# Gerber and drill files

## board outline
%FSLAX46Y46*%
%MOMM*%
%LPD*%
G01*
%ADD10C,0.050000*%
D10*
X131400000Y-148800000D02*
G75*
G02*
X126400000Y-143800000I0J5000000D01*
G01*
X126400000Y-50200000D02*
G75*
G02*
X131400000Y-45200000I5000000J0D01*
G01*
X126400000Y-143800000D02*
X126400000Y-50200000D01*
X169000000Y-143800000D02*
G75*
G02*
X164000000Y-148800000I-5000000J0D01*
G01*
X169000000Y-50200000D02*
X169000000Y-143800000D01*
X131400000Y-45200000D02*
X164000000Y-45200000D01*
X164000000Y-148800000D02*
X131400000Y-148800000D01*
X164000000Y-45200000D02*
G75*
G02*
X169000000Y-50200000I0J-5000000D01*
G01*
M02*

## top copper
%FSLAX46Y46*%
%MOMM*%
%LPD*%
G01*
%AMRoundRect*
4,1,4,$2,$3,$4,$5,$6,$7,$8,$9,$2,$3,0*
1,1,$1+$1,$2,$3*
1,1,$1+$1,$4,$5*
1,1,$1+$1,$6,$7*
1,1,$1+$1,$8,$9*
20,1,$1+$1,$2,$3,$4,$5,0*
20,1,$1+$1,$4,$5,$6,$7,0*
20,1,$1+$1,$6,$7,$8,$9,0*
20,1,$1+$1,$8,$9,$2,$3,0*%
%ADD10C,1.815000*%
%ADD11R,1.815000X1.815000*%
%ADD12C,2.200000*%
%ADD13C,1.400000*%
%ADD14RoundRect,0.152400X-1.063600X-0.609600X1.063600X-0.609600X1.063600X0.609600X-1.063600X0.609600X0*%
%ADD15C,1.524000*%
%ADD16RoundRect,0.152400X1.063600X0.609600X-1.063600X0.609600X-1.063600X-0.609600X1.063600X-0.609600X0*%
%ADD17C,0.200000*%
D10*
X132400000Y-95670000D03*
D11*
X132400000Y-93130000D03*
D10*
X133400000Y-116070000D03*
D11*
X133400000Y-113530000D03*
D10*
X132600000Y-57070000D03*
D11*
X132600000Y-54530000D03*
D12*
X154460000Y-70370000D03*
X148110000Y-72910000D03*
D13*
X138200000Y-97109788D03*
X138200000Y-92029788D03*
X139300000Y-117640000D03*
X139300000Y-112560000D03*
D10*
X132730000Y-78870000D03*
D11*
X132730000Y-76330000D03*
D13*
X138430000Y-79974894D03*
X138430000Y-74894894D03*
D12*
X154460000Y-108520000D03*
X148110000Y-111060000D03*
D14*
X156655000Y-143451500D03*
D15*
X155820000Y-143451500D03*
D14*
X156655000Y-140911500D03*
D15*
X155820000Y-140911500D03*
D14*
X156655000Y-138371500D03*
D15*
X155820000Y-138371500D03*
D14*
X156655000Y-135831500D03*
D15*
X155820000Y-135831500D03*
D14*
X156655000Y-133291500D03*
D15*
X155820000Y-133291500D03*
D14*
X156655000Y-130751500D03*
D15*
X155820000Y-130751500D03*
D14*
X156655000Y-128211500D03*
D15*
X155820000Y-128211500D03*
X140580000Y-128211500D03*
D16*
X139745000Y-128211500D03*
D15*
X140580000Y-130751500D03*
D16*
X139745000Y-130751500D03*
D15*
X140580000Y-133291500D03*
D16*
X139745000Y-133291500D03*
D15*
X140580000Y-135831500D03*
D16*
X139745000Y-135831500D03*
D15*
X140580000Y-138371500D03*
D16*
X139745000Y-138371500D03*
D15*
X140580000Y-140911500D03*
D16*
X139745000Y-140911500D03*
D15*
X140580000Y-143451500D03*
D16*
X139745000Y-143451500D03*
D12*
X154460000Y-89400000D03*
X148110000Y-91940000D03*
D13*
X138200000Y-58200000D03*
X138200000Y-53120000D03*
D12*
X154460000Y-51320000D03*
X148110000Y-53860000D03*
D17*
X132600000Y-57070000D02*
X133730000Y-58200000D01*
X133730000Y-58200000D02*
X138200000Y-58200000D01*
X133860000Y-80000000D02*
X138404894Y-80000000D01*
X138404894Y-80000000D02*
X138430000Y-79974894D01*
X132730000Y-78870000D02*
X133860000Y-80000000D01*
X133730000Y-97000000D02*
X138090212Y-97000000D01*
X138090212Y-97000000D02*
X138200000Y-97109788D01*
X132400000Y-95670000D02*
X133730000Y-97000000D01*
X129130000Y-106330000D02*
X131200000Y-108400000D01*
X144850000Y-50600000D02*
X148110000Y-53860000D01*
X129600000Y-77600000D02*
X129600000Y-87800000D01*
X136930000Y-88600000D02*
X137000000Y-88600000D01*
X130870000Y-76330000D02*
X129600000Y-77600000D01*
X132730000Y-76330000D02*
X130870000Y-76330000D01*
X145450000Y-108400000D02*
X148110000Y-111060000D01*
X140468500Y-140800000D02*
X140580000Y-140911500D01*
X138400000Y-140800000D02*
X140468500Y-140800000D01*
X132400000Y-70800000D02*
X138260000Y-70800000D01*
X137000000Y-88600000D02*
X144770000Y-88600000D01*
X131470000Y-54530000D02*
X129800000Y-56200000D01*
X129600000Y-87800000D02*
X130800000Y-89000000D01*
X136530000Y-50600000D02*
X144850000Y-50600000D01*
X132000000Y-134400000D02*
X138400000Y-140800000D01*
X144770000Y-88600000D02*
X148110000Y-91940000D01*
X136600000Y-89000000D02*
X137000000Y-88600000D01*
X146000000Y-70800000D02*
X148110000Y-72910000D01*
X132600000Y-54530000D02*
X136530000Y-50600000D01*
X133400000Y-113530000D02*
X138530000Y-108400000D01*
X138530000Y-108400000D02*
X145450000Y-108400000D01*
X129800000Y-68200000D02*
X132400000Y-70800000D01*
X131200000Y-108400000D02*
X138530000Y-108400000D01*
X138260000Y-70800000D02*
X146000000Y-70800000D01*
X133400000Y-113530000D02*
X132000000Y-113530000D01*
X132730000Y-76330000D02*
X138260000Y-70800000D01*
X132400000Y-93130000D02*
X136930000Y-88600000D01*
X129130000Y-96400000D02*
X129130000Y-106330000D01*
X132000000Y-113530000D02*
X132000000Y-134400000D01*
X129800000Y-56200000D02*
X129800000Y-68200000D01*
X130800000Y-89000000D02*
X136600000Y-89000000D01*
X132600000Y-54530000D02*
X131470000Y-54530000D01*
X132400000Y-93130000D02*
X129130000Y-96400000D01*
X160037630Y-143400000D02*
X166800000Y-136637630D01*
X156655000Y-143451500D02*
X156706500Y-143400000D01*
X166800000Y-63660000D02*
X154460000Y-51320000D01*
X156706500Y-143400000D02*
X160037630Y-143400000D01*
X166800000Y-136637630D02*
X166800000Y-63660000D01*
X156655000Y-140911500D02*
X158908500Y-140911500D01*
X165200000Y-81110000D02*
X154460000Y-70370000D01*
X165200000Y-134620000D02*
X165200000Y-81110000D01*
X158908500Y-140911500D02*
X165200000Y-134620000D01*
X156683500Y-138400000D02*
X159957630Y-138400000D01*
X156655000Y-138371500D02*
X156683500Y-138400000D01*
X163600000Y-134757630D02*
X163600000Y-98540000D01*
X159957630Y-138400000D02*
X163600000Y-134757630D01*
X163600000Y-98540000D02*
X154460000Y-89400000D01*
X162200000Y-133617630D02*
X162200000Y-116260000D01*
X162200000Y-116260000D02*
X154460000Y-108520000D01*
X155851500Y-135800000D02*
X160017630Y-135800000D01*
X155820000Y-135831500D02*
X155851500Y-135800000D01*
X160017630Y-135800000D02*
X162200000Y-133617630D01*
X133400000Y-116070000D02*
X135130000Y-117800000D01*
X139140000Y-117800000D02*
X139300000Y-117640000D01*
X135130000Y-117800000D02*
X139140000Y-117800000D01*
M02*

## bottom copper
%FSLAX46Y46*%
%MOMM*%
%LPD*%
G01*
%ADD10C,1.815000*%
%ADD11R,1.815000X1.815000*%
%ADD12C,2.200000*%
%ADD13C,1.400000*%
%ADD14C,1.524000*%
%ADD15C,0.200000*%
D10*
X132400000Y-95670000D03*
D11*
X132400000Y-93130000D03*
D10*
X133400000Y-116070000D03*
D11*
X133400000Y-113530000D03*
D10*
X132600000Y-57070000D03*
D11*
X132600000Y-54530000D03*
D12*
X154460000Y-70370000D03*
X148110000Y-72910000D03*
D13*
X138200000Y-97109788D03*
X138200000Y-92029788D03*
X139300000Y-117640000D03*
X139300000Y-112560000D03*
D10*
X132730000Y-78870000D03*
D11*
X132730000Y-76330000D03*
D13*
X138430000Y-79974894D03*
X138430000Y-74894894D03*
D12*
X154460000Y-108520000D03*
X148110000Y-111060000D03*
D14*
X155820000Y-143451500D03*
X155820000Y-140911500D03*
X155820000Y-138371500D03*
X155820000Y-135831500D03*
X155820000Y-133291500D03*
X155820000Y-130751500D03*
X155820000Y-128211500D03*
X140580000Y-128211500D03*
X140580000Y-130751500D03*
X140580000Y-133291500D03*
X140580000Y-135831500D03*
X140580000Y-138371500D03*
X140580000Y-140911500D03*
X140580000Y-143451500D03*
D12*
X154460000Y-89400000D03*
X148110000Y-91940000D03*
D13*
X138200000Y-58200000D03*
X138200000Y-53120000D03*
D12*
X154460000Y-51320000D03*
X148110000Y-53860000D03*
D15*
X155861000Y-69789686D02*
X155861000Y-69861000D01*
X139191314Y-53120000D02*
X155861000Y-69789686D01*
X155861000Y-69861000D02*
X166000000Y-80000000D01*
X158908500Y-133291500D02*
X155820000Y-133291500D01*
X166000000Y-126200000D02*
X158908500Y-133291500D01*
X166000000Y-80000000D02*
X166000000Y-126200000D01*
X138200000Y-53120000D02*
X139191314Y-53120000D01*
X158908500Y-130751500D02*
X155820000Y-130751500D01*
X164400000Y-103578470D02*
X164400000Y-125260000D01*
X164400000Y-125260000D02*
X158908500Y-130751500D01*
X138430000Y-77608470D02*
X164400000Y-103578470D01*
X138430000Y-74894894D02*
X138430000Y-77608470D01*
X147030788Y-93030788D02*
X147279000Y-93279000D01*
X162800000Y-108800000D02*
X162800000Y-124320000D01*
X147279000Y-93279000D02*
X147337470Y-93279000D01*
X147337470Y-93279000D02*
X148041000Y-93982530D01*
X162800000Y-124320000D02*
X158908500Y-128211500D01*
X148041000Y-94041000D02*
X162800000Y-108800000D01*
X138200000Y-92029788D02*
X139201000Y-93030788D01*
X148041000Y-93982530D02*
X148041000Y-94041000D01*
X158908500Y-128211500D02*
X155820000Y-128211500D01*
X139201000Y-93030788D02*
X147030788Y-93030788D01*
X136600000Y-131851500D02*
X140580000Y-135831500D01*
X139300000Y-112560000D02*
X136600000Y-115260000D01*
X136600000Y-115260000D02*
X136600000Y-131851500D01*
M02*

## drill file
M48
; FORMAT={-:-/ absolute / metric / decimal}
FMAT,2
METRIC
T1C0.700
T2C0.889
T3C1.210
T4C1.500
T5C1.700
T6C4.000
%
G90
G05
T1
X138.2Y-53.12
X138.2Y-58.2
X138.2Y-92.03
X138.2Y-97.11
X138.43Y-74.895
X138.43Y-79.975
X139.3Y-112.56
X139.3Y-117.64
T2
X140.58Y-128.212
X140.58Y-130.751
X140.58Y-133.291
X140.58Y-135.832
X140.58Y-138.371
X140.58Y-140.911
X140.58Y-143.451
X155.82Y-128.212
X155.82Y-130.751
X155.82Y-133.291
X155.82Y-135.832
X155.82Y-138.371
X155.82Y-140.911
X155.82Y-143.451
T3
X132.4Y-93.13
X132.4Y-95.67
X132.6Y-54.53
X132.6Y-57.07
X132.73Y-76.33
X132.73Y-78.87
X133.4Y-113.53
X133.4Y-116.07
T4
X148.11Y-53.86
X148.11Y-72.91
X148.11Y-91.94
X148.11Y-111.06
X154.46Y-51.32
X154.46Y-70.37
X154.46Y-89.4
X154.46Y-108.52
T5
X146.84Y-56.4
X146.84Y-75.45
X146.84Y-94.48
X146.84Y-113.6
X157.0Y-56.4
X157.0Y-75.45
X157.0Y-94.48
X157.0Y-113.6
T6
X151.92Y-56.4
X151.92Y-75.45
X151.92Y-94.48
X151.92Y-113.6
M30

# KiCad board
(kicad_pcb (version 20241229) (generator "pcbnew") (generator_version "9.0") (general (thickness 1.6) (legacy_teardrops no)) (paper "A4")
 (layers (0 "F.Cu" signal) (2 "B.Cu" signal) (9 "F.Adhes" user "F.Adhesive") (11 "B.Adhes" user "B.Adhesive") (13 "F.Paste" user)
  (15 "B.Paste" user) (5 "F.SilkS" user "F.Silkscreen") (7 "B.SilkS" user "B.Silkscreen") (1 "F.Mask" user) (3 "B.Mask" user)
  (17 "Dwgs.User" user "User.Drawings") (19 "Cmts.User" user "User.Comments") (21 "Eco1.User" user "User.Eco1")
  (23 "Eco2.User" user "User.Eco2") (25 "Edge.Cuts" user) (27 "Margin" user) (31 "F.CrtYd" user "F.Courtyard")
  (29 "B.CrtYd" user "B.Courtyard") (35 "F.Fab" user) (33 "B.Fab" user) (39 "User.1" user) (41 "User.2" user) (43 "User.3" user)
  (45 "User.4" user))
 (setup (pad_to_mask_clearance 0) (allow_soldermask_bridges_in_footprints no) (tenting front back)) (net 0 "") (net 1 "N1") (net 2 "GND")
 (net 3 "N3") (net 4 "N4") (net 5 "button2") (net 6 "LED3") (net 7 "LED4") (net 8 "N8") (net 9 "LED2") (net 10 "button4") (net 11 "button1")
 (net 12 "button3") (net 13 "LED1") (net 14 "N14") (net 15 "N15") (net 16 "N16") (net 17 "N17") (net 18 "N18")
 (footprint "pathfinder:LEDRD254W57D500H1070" (layer "F.Cu") (at 132.4 94.4 -90)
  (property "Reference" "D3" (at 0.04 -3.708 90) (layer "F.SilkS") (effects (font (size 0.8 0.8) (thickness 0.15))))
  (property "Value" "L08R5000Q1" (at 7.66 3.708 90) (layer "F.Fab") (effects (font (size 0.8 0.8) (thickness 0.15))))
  (pad "A" thru_hole circle (at 1.27 0 270) (size 1.815 1.815) (drill 1.21) (layers "*.Cu" "*.Mask") (remove_unused_layers no) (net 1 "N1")
   (solder_mask_margin 0.102))
  (pad "C" thru_hole rect (at -1.27 0 270) (size 1.815 1.815) (drill 1.21) (layers "*.Cu" "*.Mask") (remove_unused_layers no) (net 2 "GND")
   (solder_mask_margin 0.102)))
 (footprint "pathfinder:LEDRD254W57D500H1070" (layer "F.Cu") (at 133.4 114.8 -90)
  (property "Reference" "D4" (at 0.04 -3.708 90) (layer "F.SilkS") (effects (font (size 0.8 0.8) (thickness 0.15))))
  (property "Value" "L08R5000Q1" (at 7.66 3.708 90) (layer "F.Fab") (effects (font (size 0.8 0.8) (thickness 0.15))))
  (pad "A" thru_hole circle (at 1.27 0 270) (size 1.815 1.815) (drill 1.21) (layers "*.Cu" "*.Mask") (remove_unused_layers no) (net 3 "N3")
   (solder_mask_margin 0.102))
  (pad "C" thru_hole rect (at -1.27 0 270) (size 1.815 1.815) (drill 1.21) (layers "*.Cu" "*.Mask") (remove_unused_layers no) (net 2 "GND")
   (solder_mask_margin 0.102)))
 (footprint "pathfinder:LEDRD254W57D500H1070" (layer "F.Cu") (at 132.6 55.8 -90)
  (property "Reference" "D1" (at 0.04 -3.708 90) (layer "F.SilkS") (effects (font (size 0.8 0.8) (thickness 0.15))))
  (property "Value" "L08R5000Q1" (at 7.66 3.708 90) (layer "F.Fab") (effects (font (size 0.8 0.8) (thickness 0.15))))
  (pad "A" thru_hole circle (at 1.27 0 270) (size 1.815 1.815) (drill 1.21) (layers "*.Cu" "*.Mask") (remove_unused_layers no) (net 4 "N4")
   (solder_mask_margin 0.102))
  (pad "C" thru_hole rect (at -1.27 0 270) (size 1.815 1.815) (drill 1.21) (layers "*.Cu" "*.Mask") (remove_unused_layers no) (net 2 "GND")
   (solder_mask_margin 0.102)))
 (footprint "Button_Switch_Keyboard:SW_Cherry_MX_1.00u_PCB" (layer "F.Cu") (at 154.46 70.37)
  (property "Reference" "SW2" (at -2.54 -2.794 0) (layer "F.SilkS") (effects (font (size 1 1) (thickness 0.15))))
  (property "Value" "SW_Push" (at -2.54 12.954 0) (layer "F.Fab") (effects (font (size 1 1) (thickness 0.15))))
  (pad "" np_thru_hole circle (at -7.62 5.08) (size 1.7 1.7) (drill 1.7) (layers "*.Cu" "*.Mask"))
  (pad "" np_thru_hole circle (at -2.54 5.08) (size 4 4) (drill 4) (layers "*.Cu" "*.Mask"))
  (pad "" np_thru_hole circle (at 2.54 5.08) (size 1.7 1.7) (drill 1.7) (layers "*.Cu" "*.Mask"))
  (pad "1" thru_hole circle (at 0 0) (size 2.2 2.2) (drill 1.5) (layers "*.Cu" "*.Mask") (remove_unused_layers no) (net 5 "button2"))
  (pad "2" thru_hole circle (at -6.35 2.54) (size 2.2 2.2) (drill 1.5) (layers "*.Cu" "*.Mask") (remove_unused_layers no) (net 2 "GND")))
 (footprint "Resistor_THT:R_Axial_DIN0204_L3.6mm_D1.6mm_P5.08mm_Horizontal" (layer "F.Cu") (at 138.2 97.109788 90)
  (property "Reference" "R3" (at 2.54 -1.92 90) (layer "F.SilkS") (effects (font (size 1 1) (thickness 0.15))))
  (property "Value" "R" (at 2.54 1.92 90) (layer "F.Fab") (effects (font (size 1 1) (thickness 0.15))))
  (pad "1" thru_hole circle (at 0 0 90) (size 1.4 1.4) (drill 0.7) (layers "*.Cu" "*.Mask") (remove_unused_layers no) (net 1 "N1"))
  (pad "2" thru_hole circle (at 5.08 0 90) (size 1.4 1.4) (drill 0.7) (layers "*.Cu" "*.Mask") (remove_unused_layers no) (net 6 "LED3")))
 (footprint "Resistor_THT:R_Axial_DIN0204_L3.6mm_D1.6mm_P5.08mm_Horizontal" (layer "F.Cu") (at 139.3 117.64 90)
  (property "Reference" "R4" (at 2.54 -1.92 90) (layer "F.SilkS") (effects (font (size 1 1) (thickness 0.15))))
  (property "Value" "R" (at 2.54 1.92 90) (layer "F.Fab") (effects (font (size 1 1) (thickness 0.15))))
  (pad "1" thru_hole circle (at 0 0 90) (size 1.4 1.4) (drill 0.7) (layers "*.Cu" "*.Mask") (remove_unused_layers no) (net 3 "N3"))
  (pad "2" thru_hole circle (at 5.08 0 90) (size 1.4 1.4) (drill 0.7) (layers "*.Cu" "*.Mask") (remove_unused_layers no) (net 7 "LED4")))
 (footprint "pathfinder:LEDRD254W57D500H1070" (layer "F.Cu") (at 132.73 77.6 -90)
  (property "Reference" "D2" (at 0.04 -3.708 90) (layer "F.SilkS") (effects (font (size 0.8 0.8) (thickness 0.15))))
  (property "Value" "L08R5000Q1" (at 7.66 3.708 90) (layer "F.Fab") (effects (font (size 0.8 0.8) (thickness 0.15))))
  (pad "A" thru_hole circle (at 1.27 0 270) (size 1.815 1.815) (drill 1.21) (layers "*.Cu" "*.Mask") (remove_unused_layers no) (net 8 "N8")
   (solder_mask_margin 0.102))
  (pad "C" thru_hole rect (at -1.27 0 270) (size 1.815 1.815) (drill 1.21) (layers "*.Cu" "*.Mask") (remove_unused_layers no) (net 2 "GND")
   (solder_mask_margin 0.102)))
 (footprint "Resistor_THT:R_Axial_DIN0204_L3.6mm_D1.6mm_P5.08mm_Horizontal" (layer "F.Cu") (at 138.43 79.974894 90)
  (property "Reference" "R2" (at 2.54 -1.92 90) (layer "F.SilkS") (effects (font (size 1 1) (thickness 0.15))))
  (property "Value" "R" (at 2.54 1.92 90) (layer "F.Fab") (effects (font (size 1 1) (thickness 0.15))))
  (pad "1" thru_hole circle (at 0 0 90) (size 1.4 1.4) (drill 0.7) (layers "*.Cu" "*.Mask") (remove_unused_layers no) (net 8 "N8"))
  (pad "2" thru_hole circle (at 5.08 0 90) (size 1.4 1.4) (drill 0.7) (layers "*.Cu" "*.Mask") (remove_unused_layers no) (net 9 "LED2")))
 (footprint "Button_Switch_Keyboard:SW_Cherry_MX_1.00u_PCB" (layer "F.Cu") (at 154.46 108.52)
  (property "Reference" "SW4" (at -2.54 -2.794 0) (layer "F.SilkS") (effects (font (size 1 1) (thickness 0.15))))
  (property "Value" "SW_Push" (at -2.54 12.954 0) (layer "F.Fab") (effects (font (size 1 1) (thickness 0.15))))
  (pad "" np_thru_hole circle (at -7.62 5.08) (size 1.7 1.7) (drill 1.7) (layers "*.Cu" "*.Mask"))
  (pad "" np_thru_hole circle (at -2.54 5.08) (size 4 4) (drill 4) (layers "*.Cu" "*.Mask"))
  (pad "" np_thru_hole circle (at 2.54 5.08) (size 1.7 1.7) (drill 1.7) (layers "*.Cu" "*.Mask"))
  (pad "1" thru_hole circle (at 0 0) (size 2.2 2.2) (drill 1.5) (layers "*.Cu" "*.Mask") (remove_unused_layers no) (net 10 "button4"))
  (pad "2" thru_hole circle (at -6.35 2.54) (size 2.2 2.2) (drill 1.5) (layers "*.Cu" "*.Mask") (remove_unused_layers no) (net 2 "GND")))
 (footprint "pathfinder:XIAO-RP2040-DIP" (layer "F.Cu") (at 148.2 135.8315 -90)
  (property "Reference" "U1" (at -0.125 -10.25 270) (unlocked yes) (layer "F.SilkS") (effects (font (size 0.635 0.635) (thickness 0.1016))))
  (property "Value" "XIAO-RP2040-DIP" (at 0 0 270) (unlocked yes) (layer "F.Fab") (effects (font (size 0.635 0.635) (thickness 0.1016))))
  (pad "1" smd roundrect (at 7.62 -8.455) (size 2.432 1.524) (layers "F.Cu" "F.Mask") (roundrect_rratio 0.1) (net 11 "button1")
   (thermal_bridge_angle 45))
  (pad "1" thru_hole circle (at 7.62 -7.62) (size 1.524 1.524) (drill 0.889) (layers "*.Cu" "*.Mask") (remove_unused_layers no)
   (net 11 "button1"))
  (pad "2" smd roundrect (at 5.08 -8.455) (size 2.432 1.524) (layers "F.Cu" "F.Mask") (roundrect_rratio 0.1) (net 5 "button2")
   (thermal_bridge_angle 45))
  (pad "2" thru_hole circle (at 5.08 -7.62) (size 1.524 1.524) (drill 0.889) (layers "*.Cu" "*.Mask") (remove_unused_layers no)
   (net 5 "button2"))
  (pad "3" smd roundrect (at 2.54 -8.455) (size 2.432 1.524) (layers "F.Cu" "F.Mask") (roundrect_rratio 0.1) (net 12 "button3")
   (thermal_bridge_angle 45))
  (pad "3" thru_hole circle (at 2.54 -7.62) (size 1.524 1.524) (drill 0.889) (layers "*.Cu" "*.Mask") (remove_unused_layers no)
   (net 12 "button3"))
  (pad "4" smd roundrect (at 0 -8.455) (size 2.432 1.524) (layers "F.Cu" "F.Mask") (roundrect_rratio 0.1) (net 10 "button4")
   (thermal_bridge_angle 45))
  (pad "4" thru_hole circle (at 0 -7.62) (size 1.524 1.524) (drill 0.889) (layers "*.Cu" "*.Mask") (remove_unused_layers no)
   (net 10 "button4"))
  (pad "5" smd roundrect (at -2.54 -8.455) (size 2.432 1.524) (layers "F.Cu" "F.Mask") (roundrect_rratio 0.1) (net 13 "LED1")
   (thermal_bridge_angle 45))
  (pad "5" thru_hole circle (at -2.54 -7.62) (size 1.524 1.524) (drill 0.889) (layers "*.Cu" "*.Mask") (remove_unused_layers no)
   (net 13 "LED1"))
  (pad "6" smd roundrect (at -5.08 -8.455) (size 2.432 1.524) (layers "F.Cu" "F.Mask") (roundrect_rratio 0.1) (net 9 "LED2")
   (thermal_bridge_angle 45))
  (pad "6" thru_hole circle (at -5.08 -7.62) (size 1.524 1.524) (drill 0.889) (layers "*.Cu" "*.Mask") (remove_unused_layers no)
   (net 9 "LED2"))
  (pad "7" smd roundrect (at -7.62 -8.455) (size 2.432 1.524) (layers "F.Cu" "F.Mask") (roundrect_rratio 0.1) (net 6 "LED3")
   (thermal_bridge_angle 45))
  (pad "7" thru_hole circle (at -7.62 -7.62) (size 1.524 1.524) (drill 0.889) (layers "*.Cu" "*.Mask") (remove_unused_layers no)
   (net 6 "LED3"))
  (pad "8" thru_hole circle (at -7.62 7.62 180) (size 1.524 1.524) (drill 0.889) (layers "*.Cu" "*.Mask") (remove_unused_layers no)
   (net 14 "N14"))
  (pad "8" smd roundrect (at -7.62 8.455 180) (size 2.432 1.524) (layers "F.Cu" "F.Mask") (roundrect_rratio 0.1) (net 14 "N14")
   (thermal_bridge_angle 45))
  (pad "9" thru_hole circle (at -5.08 7.62 180) (size 1.524 1.524) (drill 0.889) (layers "*.Cu" "*.Mask") (remove_unused_layers no)
   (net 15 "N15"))
  (pad "9" smd roundrect (at -5.08 8.455 180) (size 2.432 1.524) (layers "F.Cu" "F.Mask") (roundrect_rratio 0.1) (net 15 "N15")
   (thermal_bridge_angle 45))
  (pad "10" thru_hole circle (at -2.54 7.62 180) (size 1.524 1.524) (drill 0.889) (layers "*.Cu" "*.Mask") (remove_unused_layers no)
   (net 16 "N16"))
  (pad "10" smd roundrect (at -2.54 8.455 180) (size 2.432 1.524) (layers "F.Cu" "F.Mask") (roundrect_rratio 0.1) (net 16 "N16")
   (thermal_bridge_angle 45))
  (pad "11" thru_hole circle (at 0 7.62 180) (size 1.524 1.524) (drill 0.889) (layers "*.Cu" "*.Mask") (remove_unused_layers no)
   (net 7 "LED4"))
  (pad "11" smd roundrect (at 0 8.455 180) (size 2.432 1.524) (layers "F.Cu" "F.Mask") (roundrect_rratio 0.1) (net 7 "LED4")
   (thermal_bridge_angle 45))
  (pad "12" thru_hole circle (at 2.54 7.62 180) (size 1.524 1.524) (drill 0.889) (layers "*.Cu" "*.Mask") (remove_unused_layers no)
   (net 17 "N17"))
  (pad "12" smd roundrect (at 2.54 8.455 180) (size 2.432 1.524) (layers "F.Cu" "F.Mask") (roundrect_rratio 0.1) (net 17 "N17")
   (thermal_bridge_angle 45))
  (pad "13" thru_hole circle (at 5.08 7.62 180) (size 1.524 1.524) (drill 0.889) (layers "*.Cu" "*.Mask") (remove_unused_layers no)
   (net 2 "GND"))
  (pad "13" smd roundrect (at 5.08 8.455 180) (size 2.432 1.524) (layers "F.Cu" "F.Mask") (roundrect_rratio 0.1) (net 2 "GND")
   (thermal_bridge_angle 45))
  (pad "14" thru_hole circle (at 7.62 7.62 180) (size 1.524 1.524) (drill 0.889) (layers "*.Cu" "*.Mask") (remove_unused_layers no)
   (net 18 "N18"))
  (pad "14" smd roundrect (at 7.62 8.455 180) (size 2.432 1.524) (layers "F.Cu" "F.Mask") (roundrect_rratio 0.1) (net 18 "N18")
   (thermal_bridge_angle 45)))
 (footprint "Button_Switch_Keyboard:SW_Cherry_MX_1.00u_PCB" (layer "F.Cu") (at 154.46 89.4)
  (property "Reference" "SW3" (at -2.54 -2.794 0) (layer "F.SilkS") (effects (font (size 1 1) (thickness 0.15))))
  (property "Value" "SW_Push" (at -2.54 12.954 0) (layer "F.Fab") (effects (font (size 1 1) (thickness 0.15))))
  (pad "" np_thru_hole circle (at -7.62 5.08) (size 1.7 1.7) (drill 1.7) (layers "*.Cu" "*.Mask"))
  (pad "" np_thru_hole circle (at -2.54 5.08) (size 4 4) (drill 4) (layers "*.Cu" "*.Mask"))
  (pad "" np_thru_hole circle (at 2.54 5.08) (size 1.7 1.7) (drill 1.7) (layers "*.Cu" "*.Mask"))
  (pad "1" thru_hole circle (at 0 0) (size 2.2 2.2) (drill 1.5) (layers "*.Cu" "*.Mask") (remove_unused_layers no) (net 12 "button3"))
  (pad "2" thru_hole circle (at -6.35 2.54) (size 2.2 2.2) (drill 1.5) (layers "*.Cu" "*.Mask") (remove_unused_layers no) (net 2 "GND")))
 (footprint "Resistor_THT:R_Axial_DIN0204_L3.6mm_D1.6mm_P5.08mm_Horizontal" (layer "F.Cu") (at 138.2 58.2 90)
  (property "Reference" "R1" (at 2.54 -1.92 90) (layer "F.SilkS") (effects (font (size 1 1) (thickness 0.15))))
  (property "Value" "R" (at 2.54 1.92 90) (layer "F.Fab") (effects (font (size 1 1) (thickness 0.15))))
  (pad "1" thru_hole circle (at 0 0 90) (size 1.4 1.4) (drill 0.7) (layers "*.Cu" "*.Mask") (remove_unused_layers no) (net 4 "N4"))
  (pad "2" thru_hole circle (at 5.08 0 90) (size 1.4 1.4) (drill 0.7) (layers "*.Cu" "*.Mask") (remove_unused_layers no) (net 13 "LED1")))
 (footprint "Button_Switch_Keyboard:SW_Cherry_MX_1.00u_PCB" (layer "F.Cu") (at 154.46 51.32)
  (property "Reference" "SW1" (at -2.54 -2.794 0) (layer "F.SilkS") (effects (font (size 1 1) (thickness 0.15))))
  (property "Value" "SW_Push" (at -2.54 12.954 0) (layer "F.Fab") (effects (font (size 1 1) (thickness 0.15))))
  (pad "" np_thru_hole circle (at -7.62 5.08) (size 1.7 1.7) (drill 1.7) (layers "*.Cu" "*.Mask"))
  (pad "" np_thru_hole circle (at -2.54 5.08) (size 4 4) (drill 4) (layers "*.Cu" "*.Mask"))
  (pad "" np_thru_hole circle (at 2.54 5.08) (size 1.7 1.7) (drill 1.7) (layers "*.Cu" "*.Mask"))
  (pad "1" thru_hole circle (at 0 0) (size 2.2 2.2) (drill 1.5) (layers "*.Cu" "*.Mask") (remove_unused_layers no) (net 11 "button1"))
  (pad "2" thru_hole circle (at -6.35 2.54) (size 2.2 2.2) (drill 1.5) (layers "*.Cu" "*.Mask") (remove_unused_layers no) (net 2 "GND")))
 (gr_arc (start 131.4 148.8) (mid 127.864466 147.335534) (end 126.4 143.8) (stroke (width 0.05) (type default)) (layer "Edge.Cuts"))
 (gr_arc (start 126.4 50.2) (mid 127.864466 46.664466) (end 131.4 45.2) (stroke (width 0.05) (type default)) (layer "Edge.Cuts"))
 (gr_line (start 126.4 143.8) (end 126.4 50.2) (stroke (width 0.05) (type default)) (layer "Edge.Cuts"))
 (gr_arc (start 169 143.8) (mid 167.535534 147.335534) (end 164 148.8) (stroke (width 0.05) (type default)) (layer "Edge.Cuts"))
 (gr_line (start 169 50.2) (end 169 143.8) (stroke (width 0.05) (type default)) (layer "Edge.Cuts"))
 (gr_line (start 131.4 45.2) (end 164 45.2) (stroke (width 0.05) (type default)) (layer "Edge.Cuts"))
 (gr_line (start 164 148.8) (end 131.4 148.8) (stroke (width 0.05) (type default)) (layer "Edge.Cuts"))
 (gr_arc (start 164 45.2) (mid 167.535534 46.664466) (end 169 50.2) (stroke (width 0.05) (type default)) (layer "Edge.Cuts"))
 (segment (start 155.861 69.789686) (end 155.861 69.861) (width 0.2) (layer "B.Cu") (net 13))
 (segment (start 139.191314 53.12) (end 155.861 69.789686) (width 0.2) (layer "B.Cu") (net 13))
 (segment (start 155.861 69.861) (end 166 80) (width 0.2) (layer "B.Cu") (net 13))
 (segment (start 158.9085 133.2915) (end 155.82 133.2915) (width 0.2) (layer "B.Cu") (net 13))
 (segment (start 166 126.2) (end 158.9085 133.2915) (width 0.2) (layer "B.Cu") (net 13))
 (segment (start 166 80) (end 166 126.2) (width 0.2) (layer "B.Cu") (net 13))
 (segment (start 138.2 53.12) (end 139.191314 53.12) (width 0.2) (layer "B.Cu") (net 13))
 (segment (start 132.6 57.07) (end 133.73 58.2) (width 0.2) (layer "F.Cu") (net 4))
 (segment (start 133.73 58.2) (end 138.2 58.2) (width 0.2) (layer "F.Cu") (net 4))
 (segment (start 133.86 80) (end 138.404894 80) (width 0.2) (layer "F.Cu") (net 8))
 (segment (start 138.404894 80) (end 138.43 79.974894) (width 0.2) (layer "F.Cu") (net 8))
 (segment (start 132.73 78.87) (end 133.86 80) (width 0.2) (layer "F.Cu") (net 8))
 (segment (start 158.9085 130.7515) (end 155.82 130.7515) (width 0.2) (layer "B.Cu") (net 9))
 (segment (start 164.4 103.57847) (end 164.4 125.26) (width 0.2) (layer "B.Cu") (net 9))
 (segment (start 164.4 125.26) (end 158.9085 130.7515) (width 0.2) (layer "B.Cu") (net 9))
 (segment (start 138.43 77.60847) (end 164.4 103.57847) (width 0.2) (layer "B.Cu") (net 9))
 (segment (start 138.43 74.894894) (end 138.43 77.60847) (width 0.2) (layer "B.Cu") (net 9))
 (segment (start 147.030788 93.030788) (end 147.279 93.279) (width 0.2) (layer "B.Cu") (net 6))
 (segment (start 162.8 108.8) (end 162.8 124.32) (width 0.2) (layer "B.Cu") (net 6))
 (segment (start 147.279 93.279) (end 147.33747 93.279) (width 0.2) (layer "B.Cu") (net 6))
 (segment (start 147.33747 93.279) (end 148.041 93.98253) (width 0.2) (layer "B.Cu") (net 6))
 (segment (start 162.8 124.32) (end 158.9085 128.2115) (width 0.2) (layer "B.Cu") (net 6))
 (segment (start 148.041 94.041) (end 162.8 108.8) (width 0.2) (layer "B.Cu") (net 6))
 (segment (start 138.2 92.029788) (end 139.201 93.030788) (width 0.2) (layer "B.Cu") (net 6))
 (segment (start 148.041 93.98253) (end 148.041 94.041) (width 0.2) (layer "B.Cu") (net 6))
 (segment (start 158.9085 128.2115) (end 155.82 128.2115) (width 0.2) (layer "B.Cu") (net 6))
 (segment (start 139.201 93.030788) (end 147.030788 93.030788) (width 0.2) (layer "B.Cu") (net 6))
 (segment (start 133.73 97) (end 138.090212 97) (width 0.2) (layer "F.Cu") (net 1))
 (segment (start 138.090212 97) (end 138.2 97.109788) (width 0.2) (layer "F.Cu") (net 1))
 (segment (start 132.4 95.67) (end 133.73 97) (width 0.2) (layer "F.Cu") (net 1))
 (segment (start 129.13 106.33) (end 131.2 108.4) (width 0.2) (layer "F.Cu") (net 2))
 (segment (start 144.85 50.6) (end 148.11 53.86) (width 0.2) (layer "F.Cu") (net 2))
 (segment (start 129.6 77.6) (end 129.6 87.8) (width 0.2) (layer "F.Cu") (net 2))
 (segment (start 136.93 88.6) (end 137 88.6) (width 0.2) (layer "F.Cu") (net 2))
 (segment (start 130.87 76.33) (end 129.6 77.6) (width 0.2) (layer "F.Cu") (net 2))
 (segment (start 132.73 76.33) (end 130.87 76.33) (width 0.2) (layer "F.Cu") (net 2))
 (segment (start 145.45 108.4) (end 148.11 111.06) (width 0.2) (layer "F.Cu") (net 2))
 (segment (start 140.4685 140.8) (end 140.58 140.9115) (width 0.2) (layer "F.Cu") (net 2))
 (segment (start 138.4 140.8) (end 140.4685 140.8) (width 0.2) (layer "F.Cu") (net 2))
 (segment (start 132.4 70.8) (end 138.26 70.8) (width 0.2) (layer "F.Cu") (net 2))
 (segment (start 137 88.6) (end 144.77 88.6) (width 0.2) (layer "F.Cu") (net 2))
 (segment (start 131.47 54.53) (end 129.8 56.2) (width 0.2) (layer "F.Cu") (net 2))
 (segment (start 129.6 87.8) (end 130.8 89) (width 0.2) (layer "F.Cu") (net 2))
 (segment (start 136.53 50.6) (end 144.85 50.6) (width 0.2) (layer "F.Cu") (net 2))
 (segment (start 132 134.4) (end 138.4 140.8) (width 0.2) (layer "F.Cu") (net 2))
 (segment (start 144.77 88.6) (end 148.11 91.94) (width 0.2) (layer "F.Cu") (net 2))
 (segment (start 136.6 89) (end 137 88.6) (width 0.2) (layer "F.Cu") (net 2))
 (segment (start 146 70.8) (end 148.11 72.91) (width 0.2) (layer "F.Cu") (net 2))
 (segment (start 132.6 54.53) (end 136.53 50.6) (width 0.2) (layer "F.Cu") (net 2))
 (segment (start 133.4 113.53) (end 138.53 108.4) (width 0.2) (layer "F.Cu") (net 2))
 (segment (start 138.53 108.4) (end 145.45 108.4) (width 0.2) (layer "F.Cu") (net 2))
 (segment (start 129.8 68.2) (end 132.4 70.8) (width 0.2) (layer "F.Cu") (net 2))
 (segment (start 131.2 108.4) (end 138.53 108.4) (width 0.2) (layer "F.Cu") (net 2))
 (segment (start 138.26 70.8) (end 146 70.8) (width 0.2) (layer "F.Cu") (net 2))
 (segment (start 133.4 113.53) (end 132 113.53) (width 0.2) (layer "F.Cu") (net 2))
 (segment (start 132.73 76.33) (end 138.26 70.8) (width 0.2) (layer "F.Cu") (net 2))
 (segment (start 132.4 93.13) (end 136.93 88.6) (width 0.2) (layer "F.Cu") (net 2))
 (segment (start 129.13 96.4) (end 129.13 106.33) (width 0.2) (layer "F.Cu") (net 2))
 (segment (start 132 113.53) (end 132 134.4) (width 0.2) (layer "F.Cu") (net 2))
 (segment (start 129.8 56.2) (end 129.8 68.2) (width 0.2) (layer "F.Cu") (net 2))
 (segment (start 130.8 89) (end 136.6 89) (width 0.2) (layer "F.Cu") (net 2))
 (segment (start 132.6 54.53) (end 131.47 54.53) (width 0.2) (layer "F.Cu") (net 2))
 (segment (start 132.4 93.13) (end 129.13 96.4) (width 0.2) (layer "F.Cu") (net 2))
 (segment (start 160.03763 143.4) (end 166.8 136.63763) (width 0.2) (layer "F.Cu") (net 11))
 (segment (start 156.655 143.4515) (end 156.7065 143.4) (width 0.2) (layer "F.Cu") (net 11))
 (segment (start 166.8 63.66) (end 154.46 51.32) (width 0.2) (layer "F.Cu") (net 11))
 (segment (start 156.7065 143.4) (end 160.03763 143.4) (width 0.2) (layer "F.Cu") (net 11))
 (segment (start 166.8 136.63763) (end 166.8 63.66) (width 0.2) (layer "F.Cu") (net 11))
 (segment (start 156.655 140.9115) (end 158.9085 140.9115) (width 0.2) (layer "F.Cu") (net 5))
 (segment (start 165.2 81.11) (end 154.46 70.37) (width 0.2) (layer "F.Cu") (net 5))
 (segment (start 165.2 134.62) (end 165.2 81.11) (width 0.2) (layer "F.Cu") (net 5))
 (segment (start 158.9085 140.9115) (end 165.2 134.62) (width 0.2) (layer "F.Cu") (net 5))
 (segment (start 156.6835 138.4) (end 159.95763 138.4) (width 0.2) (layer "F.Cu") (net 12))
 (segment (start 156.655 138.3715) (end 156.6835 138.4) (width 0.2) (layer "F.Cu") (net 12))
 (segment (start 163.6 134.75763) (end 163.6 98.54) (width 0.2) (layer "F.Cu") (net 12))
 (segment (start 159.95763 138.4) (end 163.6 134.75763) (width 0.2) (layer "F.Cu") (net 12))
 (segment (start 163.6 98.54) (end 154.46 89.4) (width 0.2) (layer "F.Cu") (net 12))
 (segment (start 136.6 131.8515) (end 140.58 135.8315) (width 0.2) (layer "B.Cu") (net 7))
 (segment (start 139.3 112.56) (end 136.6 115.26) (width 0.2) (layer "B.Cu") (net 7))
 (segment (start 136.6 115.26) (end 136.6 131.8515) (width 0.2) (layer "B.Cu") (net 7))
 (segment (start 162.2 133.61763) (end 162.2 116.26) (width 0.2) (layer "F.Cu") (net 10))
 (segment (start 162.2 116.26) (end 154.46 108.52) (width 0.2) (layer "F.Cu") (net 10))
 (segment (start 155.8515 135.8) (end 160.01763 135.8) (width 0.2) (layer "F.Cu") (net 10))
 (segment (start 155.82 135.8315) (end 155.8515 135.8) (width 0.2) (layer "F.Cu") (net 10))
 (segment (start 160.01763 135.8) (end 162.2 133.61763) (width 0.2) (layer "F.Cu") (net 10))
 (segment (start 133.4 116.07) (end 135.13 117.8) (width 0.2) (layer "F.Cu") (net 3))
 (segment (start 139.14 117.8) (end 139.3 117.64) (width 0.2) (layer "F.Cu") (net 3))
 (segment (start 135.13 117.8) (end 139.14 117.8) (width 0.2) (layer "F.Cu") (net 3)))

